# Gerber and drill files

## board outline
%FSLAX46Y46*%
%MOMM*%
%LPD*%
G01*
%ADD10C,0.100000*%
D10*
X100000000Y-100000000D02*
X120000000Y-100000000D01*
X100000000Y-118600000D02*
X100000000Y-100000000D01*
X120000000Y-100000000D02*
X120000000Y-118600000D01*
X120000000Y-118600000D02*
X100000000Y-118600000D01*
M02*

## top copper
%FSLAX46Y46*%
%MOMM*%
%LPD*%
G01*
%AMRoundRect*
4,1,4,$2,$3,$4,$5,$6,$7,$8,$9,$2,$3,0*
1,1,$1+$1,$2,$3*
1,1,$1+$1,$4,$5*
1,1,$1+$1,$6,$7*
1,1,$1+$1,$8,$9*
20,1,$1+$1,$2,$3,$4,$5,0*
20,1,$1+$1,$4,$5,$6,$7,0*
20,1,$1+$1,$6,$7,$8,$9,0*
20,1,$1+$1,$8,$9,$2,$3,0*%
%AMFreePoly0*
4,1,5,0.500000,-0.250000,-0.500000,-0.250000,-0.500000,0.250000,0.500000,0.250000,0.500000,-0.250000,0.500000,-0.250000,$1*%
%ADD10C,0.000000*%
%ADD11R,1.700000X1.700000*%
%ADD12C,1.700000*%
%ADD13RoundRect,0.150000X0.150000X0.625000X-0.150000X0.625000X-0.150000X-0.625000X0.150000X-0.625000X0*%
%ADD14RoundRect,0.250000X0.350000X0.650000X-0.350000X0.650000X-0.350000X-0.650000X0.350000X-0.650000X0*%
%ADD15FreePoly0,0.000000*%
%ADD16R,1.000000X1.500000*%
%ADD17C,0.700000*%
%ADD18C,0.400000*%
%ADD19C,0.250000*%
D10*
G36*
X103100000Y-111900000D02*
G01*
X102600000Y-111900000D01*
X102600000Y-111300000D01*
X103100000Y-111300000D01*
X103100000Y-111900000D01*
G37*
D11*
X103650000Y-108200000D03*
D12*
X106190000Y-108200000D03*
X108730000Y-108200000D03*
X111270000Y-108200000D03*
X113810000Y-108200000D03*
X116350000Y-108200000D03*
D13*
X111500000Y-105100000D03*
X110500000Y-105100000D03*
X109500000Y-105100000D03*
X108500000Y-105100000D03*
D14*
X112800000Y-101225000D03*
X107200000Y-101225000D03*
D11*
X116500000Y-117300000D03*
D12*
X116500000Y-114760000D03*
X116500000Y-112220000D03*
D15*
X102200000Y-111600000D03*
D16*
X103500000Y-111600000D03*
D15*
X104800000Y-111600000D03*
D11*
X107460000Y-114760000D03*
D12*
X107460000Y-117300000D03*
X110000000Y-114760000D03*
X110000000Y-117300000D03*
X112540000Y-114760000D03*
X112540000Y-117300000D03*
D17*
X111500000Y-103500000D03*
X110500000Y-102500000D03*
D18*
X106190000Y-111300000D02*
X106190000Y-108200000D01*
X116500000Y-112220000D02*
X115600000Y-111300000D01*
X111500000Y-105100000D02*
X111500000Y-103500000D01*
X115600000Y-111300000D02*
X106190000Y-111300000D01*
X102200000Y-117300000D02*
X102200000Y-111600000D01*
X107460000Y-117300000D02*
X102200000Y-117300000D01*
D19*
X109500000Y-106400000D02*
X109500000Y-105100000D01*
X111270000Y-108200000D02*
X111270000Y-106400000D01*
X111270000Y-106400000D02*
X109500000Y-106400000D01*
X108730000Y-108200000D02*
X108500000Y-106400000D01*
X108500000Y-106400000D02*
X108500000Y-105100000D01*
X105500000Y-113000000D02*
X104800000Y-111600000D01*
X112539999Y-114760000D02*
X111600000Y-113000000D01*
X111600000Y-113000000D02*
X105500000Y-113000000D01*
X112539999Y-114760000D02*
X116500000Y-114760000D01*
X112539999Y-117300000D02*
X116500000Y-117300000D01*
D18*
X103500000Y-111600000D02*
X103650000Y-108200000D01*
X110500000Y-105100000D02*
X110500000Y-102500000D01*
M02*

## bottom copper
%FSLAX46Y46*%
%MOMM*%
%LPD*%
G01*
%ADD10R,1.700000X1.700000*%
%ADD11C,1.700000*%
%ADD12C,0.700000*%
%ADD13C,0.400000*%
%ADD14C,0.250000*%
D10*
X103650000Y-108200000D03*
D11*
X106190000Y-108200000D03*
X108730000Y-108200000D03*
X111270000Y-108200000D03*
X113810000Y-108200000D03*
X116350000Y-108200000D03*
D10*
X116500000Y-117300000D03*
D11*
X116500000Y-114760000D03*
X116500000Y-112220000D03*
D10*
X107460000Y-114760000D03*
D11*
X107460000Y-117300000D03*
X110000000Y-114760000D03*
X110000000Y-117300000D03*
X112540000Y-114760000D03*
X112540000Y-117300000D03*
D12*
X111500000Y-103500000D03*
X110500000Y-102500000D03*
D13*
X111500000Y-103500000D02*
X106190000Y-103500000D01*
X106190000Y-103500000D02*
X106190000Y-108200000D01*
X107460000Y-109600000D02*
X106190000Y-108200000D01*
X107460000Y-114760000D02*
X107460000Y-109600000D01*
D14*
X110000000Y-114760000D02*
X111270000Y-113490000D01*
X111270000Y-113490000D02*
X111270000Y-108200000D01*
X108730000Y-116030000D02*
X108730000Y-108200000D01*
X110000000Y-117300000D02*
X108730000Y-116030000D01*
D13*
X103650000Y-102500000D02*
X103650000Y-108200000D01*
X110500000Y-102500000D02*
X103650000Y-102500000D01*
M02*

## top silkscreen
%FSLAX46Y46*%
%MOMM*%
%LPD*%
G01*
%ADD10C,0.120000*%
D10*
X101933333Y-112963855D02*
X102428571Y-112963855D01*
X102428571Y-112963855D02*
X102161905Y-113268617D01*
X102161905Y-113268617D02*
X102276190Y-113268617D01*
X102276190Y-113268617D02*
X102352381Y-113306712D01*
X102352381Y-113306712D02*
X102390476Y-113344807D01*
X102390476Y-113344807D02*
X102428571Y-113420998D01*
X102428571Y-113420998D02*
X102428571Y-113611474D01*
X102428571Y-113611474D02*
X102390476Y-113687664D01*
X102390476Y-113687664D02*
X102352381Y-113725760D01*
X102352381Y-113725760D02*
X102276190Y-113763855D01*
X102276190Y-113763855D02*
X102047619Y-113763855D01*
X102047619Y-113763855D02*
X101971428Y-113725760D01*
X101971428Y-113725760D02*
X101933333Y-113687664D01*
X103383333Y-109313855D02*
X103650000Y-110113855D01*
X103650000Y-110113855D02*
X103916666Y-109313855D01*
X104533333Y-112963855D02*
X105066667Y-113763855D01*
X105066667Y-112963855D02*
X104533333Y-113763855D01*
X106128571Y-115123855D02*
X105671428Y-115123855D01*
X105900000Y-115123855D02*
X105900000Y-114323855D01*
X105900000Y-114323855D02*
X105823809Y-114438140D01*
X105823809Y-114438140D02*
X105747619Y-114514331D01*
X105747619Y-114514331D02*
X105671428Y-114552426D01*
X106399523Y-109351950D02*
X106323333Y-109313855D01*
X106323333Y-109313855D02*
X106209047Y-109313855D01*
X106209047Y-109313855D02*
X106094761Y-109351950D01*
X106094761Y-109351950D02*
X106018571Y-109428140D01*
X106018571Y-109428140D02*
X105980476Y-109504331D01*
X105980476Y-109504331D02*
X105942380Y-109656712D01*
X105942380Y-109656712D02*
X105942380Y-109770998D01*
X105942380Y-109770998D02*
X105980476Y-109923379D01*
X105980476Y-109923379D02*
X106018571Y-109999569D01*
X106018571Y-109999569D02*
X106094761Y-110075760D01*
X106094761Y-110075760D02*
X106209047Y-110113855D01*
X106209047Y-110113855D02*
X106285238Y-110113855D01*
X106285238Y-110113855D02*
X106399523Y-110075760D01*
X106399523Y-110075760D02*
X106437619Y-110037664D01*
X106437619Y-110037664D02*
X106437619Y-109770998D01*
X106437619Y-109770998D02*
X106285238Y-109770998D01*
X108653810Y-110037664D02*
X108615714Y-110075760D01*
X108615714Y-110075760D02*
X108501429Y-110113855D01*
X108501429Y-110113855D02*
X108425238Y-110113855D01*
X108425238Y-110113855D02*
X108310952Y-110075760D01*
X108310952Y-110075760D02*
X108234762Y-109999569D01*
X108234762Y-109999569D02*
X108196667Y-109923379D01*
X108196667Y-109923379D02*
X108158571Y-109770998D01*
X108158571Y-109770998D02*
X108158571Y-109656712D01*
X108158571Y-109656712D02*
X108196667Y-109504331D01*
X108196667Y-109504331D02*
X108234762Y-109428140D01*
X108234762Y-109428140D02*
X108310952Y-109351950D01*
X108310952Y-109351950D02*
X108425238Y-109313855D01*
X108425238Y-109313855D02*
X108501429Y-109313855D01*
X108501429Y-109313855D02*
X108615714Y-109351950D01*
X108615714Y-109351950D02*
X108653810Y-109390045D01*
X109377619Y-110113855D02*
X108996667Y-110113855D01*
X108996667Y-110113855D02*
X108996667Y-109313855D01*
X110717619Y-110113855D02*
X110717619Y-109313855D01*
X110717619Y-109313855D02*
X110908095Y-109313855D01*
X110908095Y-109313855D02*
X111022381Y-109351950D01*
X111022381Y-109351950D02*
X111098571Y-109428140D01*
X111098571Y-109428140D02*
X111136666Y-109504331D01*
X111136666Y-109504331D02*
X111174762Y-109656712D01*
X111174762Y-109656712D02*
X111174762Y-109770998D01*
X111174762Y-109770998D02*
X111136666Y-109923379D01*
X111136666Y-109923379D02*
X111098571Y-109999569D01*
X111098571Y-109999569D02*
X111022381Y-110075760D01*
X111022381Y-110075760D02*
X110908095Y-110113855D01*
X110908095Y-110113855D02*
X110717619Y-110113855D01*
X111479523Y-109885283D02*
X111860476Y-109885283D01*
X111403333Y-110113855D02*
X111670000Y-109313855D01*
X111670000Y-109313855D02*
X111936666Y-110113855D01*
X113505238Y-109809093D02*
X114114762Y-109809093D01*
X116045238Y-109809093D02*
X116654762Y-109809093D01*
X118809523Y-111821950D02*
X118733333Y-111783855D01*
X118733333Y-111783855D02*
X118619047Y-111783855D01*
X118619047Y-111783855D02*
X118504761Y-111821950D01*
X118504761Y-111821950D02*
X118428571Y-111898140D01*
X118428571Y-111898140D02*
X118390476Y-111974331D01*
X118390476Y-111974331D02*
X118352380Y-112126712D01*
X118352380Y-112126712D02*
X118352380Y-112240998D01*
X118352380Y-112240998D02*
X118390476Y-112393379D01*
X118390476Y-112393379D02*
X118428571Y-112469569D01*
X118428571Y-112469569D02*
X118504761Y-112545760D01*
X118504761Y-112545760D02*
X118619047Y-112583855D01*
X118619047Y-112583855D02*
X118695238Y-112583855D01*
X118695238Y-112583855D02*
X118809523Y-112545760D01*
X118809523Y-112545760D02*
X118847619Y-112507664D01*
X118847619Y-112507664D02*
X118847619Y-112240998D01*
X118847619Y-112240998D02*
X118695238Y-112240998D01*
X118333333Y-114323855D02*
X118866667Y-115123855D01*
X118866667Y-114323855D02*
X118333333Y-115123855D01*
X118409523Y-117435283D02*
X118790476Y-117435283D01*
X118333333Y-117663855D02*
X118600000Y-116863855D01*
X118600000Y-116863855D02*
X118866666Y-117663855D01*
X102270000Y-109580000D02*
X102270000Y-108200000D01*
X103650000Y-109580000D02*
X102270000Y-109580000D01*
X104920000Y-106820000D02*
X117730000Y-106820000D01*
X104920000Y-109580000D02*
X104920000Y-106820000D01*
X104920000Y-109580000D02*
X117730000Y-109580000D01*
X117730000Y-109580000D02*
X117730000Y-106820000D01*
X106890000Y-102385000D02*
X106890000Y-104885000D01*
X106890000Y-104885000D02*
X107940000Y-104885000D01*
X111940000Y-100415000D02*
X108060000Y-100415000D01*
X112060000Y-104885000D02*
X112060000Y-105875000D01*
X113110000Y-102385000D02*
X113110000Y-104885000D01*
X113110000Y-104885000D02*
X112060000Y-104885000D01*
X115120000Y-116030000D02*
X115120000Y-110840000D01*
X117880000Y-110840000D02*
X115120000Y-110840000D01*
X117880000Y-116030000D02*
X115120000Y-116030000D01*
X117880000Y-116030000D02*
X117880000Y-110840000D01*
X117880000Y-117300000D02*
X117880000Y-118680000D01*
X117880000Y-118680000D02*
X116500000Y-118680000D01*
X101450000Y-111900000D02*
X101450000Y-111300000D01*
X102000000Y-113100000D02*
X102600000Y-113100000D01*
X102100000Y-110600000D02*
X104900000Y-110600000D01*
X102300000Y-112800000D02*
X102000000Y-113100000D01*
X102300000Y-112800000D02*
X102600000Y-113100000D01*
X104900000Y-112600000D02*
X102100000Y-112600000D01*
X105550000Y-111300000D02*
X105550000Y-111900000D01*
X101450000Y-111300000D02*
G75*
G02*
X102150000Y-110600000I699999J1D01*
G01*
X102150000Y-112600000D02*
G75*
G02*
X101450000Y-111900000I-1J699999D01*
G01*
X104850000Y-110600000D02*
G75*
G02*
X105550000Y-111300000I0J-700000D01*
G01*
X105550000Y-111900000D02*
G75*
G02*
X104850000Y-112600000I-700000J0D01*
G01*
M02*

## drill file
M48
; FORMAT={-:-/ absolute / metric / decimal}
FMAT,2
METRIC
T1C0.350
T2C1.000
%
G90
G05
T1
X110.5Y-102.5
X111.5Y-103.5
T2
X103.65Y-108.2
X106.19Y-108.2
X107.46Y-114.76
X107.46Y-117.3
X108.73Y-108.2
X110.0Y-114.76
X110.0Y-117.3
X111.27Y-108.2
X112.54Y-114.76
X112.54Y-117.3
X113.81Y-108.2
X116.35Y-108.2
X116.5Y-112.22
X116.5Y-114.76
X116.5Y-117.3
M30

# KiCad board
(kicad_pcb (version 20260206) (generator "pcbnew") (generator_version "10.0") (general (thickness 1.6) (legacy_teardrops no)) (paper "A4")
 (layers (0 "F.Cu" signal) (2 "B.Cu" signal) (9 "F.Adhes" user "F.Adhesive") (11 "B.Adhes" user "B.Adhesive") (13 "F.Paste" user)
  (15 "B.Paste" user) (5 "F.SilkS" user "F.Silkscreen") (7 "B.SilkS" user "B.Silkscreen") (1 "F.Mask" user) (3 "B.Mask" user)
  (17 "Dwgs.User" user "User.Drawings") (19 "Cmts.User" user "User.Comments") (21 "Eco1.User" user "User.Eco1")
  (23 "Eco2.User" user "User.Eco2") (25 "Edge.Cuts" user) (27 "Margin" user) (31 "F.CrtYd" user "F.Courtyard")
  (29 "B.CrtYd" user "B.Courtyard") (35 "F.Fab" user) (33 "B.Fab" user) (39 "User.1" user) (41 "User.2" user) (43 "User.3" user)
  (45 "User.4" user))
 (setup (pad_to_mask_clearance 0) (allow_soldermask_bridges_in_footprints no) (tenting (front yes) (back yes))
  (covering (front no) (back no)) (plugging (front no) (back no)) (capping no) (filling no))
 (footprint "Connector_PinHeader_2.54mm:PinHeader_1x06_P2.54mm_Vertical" (layer "F.Cu") (at 103.65 108.2 90)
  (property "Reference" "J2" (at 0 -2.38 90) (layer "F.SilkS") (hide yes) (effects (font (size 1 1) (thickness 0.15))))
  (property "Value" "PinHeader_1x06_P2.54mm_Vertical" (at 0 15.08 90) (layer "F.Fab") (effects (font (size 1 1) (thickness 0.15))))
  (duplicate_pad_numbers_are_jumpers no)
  (fp_line (start -1.38 -1.38) (end 0 -1.38) (stroke (width 0.12) (type solid)) (layer "F.SilkS"))
  (fp_line (start -1.38 0) (end -1.38 -1.38) (stroke (width 0.12) (type solid)) (layer "F.SilkS"))
  (fp_line (start 1.38 1.27) (end 1.38 14.08) (stroke (width 0.12) (type solid)) (layer "F.SilkS"))
  (fp_line (start -1.38 1.27) (end 1.38 1.27) (stroke (width 0.12) (type solid)) (layer "F.SilkS"))
  (fp_line (start -1.38 1.27) (end -1.38 14.08) (stroke (width 0.12) (type solid)) (layer "F.SilkS"))
  (fp_line (start -1.38 14.08) (end 1.38 14.08) (stroke (width 0.12) (type solid)) (layer "F.SilkS"))
  (pad "1" thru_hole rect (at 0 0 90) (size 1.7 1.7) (drill 1) (layers "*.Cu" "*.Mask") (remove_unused_layers no) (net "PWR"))
  (pad "2" thru_hole circle (at 0 2.54 90) (size 1.7 1.7) (drill 1) (layers "*.Cu" "*.Mask") (remove_unused_layers no) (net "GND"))
  (pad "3" thru_hole circle (at 0 5.08 90) (size 1.7 1.7) (drill 1) (layers "*.Cu" "*.Mask") (remove_unused_layers no) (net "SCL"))
  (pad "4" thru_hole circle (at 0 7.62 90) (size 1.7 1.7) (drill 1) (layers "*.Cu" "*.Mask") (remove_unused_layers no) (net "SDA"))
  (pad "5" thru_hole circle (at 0 10.16 90) (size 1.7 1.7) (drill 1) (layers "*.Cu" "*.Mask") (remove_unused_layers no))
  (pad "6" thru_hole circle (at 0 12.7 90) (size 1.7 1.7) (drill 1) (layers "*.Cu" "*.Mask") (remove_unused_layers no)))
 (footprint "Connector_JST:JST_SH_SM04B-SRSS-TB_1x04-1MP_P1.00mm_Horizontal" (layer "F.Cu") (at 110 103.1 180)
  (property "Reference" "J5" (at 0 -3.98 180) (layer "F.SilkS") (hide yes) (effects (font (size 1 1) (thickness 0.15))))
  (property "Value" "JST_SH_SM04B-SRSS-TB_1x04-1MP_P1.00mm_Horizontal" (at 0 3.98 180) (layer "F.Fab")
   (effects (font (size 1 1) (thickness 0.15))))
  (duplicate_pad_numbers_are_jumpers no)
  (fp_line (start 3.11 0.715) (end 3.11 -1.785) (stroke (width 0.12) (type solid)) (layer "F.SilkS"))
  (fp_line (start 3.11 -1.785) (end 2.06 -1.785) (stroke (width 0.12) (type solid)) (layer "F.SilkS"))
  (fp_line (start -1.94 2.685) (end 1.94 2.685) (stroke (width 0.12) (type solid)) (layer "F.SilkS"))
  (fp_line (start -2.06 -1.785) (end -2.06 -2.775) (stroke (width 0.12) (type solid)) (layer "F.SilkS"))
  (fp_line (start -3.11 0.715) (end -3.11 -1.785) (stroke (width 0.12) (type solid)) (layer "F.SilkS"))
  (fp_line (start -3.11 -1.785) (end -2.06 -1.785) (stroke (width 0.12) (type solid)) (layer "F.SilkS"))
  (pad "1" smd roundrect (at -1.5 -2 180) (size 0.6 1.55) (layers "F.Cu" "F.Mask" "F.Paste") (roundrect_rratio 0.25) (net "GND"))
  (pad "2" smd roundrect (at -0.5 -2 180) (size 0.6 1.55) (layers "F.Cu" "F.Mask" "F.Paste") (roundrect_rratio 0.25) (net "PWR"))
  (pad "3" smd roundrect (at 0.5 -2 180) (size 0.6 1.55) (layers "F.Cu" "F.Mask" "F.Paste") (roundrect_rratio 0.25) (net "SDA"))
  (pad "4" smd roundrect (at 1.5 -2 180) (size 0.6 1.55) (layers "F.Cu" "F.Mask" "F.Paste") (roundrect_rratio 0.25) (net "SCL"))
  (pad "MP" smd roundrect (at -2.8 1.875 180) (size 1.2 1.8) (layers "F.Cu" "F.Mask" "F.Paste") (roundrect_rratio 0.208333))
  (pad "MP" smd roundrect (at 2.8 1.875 180) (size 1.2 1.8) (layers "F.Cu" "F.Mask" "F.Paste") (roundrect_rratio 0.208333)))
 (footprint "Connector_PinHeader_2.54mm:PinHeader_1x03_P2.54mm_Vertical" (layer "F.Cu") (at 116.5 117.3 180)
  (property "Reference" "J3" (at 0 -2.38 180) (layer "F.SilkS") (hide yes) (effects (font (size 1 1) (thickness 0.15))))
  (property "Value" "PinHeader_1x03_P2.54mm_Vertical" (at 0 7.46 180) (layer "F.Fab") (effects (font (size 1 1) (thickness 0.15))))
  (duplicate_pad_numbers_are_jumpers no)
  (fp_line (start 1.38 1.27) (end 1.38 6.46) (stroke (width 0.12) (type solid)) (layer "F.SilkS"))
  (fp_line (start -1.38 6.46) (end 1.38 6.46) (stroke (width 0.12) (type solid)) (layer "F.SilkS"))
  (fp_line (start -1.38 1.27) (end 1.38 1.27) (stroke (width 0.12) (type solid)) (layer "F.SilkS"))
  (fp_line (start -1.38 1.27) (end -1.38 6.46) (stroke (width 0.12) (type solid)) (layer "F.SilkS"))
  (fp_line (start -1.38 0) (end -1.38 -1.38) (stroke (width 0.12) (type solid)) (layer "F.SilkS"))
  (fp_line (start -1.38 -1.38) (end 0 -1.38) (stroke (width 0.12) (type solid)) (layer "F.SilkS"))
  (pad "1" thru_hole rect (at 0 0 180) (size 1.7 1.7) (drill 1) (layers "*.Cu" "*.Mask") (remove_unused_layers no) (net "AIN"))
  (pad "2" thru_hole circle (at 0 2.54 180) (size 1.7 1.7) (drill 1) (layers "*.Cu" "*.Mask") (remove_unused_layers no) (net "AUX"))
  (pad "3" thru_hole circle (at 0 5.08 180) (size 1.7 1.7) (drill 1) (layers "*.Cu" "*.Mask") (remove_unused_layers no) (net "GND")))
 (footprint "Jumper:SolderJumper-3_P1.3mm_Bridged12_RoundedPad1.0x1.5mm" (layer "F.Cu") (at 103.5 111.6)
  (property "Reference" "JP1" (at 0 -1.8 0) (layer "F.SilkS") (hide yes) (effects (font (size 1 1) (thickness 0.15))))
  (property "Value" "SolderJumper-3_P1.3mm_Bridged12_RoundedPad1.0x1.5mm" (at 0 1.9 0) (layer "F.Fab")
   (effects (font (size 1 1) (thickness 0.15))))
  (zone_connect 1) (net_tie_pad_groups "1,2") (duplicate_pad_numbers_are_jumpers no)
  (fp_poly (pts (xy -0.9 -0.3) (xy -0.4 -0.3) (xy -0.4 0.3) (xy -0.9 0.3)) (stroke (width 0) (type solid)) (fill yes) (layer "F.Cu"))
  (fp_line (start -2.05 0.3) (end -2.05 -0.3) (stroke (width 0.12) (type solid)) (layer "F.SilkS"))
  (fp_line (start -1.5 1.5) (end -0.9 1.5) (stroke (width 0.12) (type solid)) (layer "F.SilkS"))
  (fp_line (start -1.4 -1) (end 1.4 -1) (stroke (width 0.12) (type solid)) (layer "F.SilkS"))
  (fp_line (start -1.2 1.2) (end -1.5 1.5) (stroke (width 0.12) (type solid)) (layer "F.SilkS"))
  (fp_line (start -1.2 1.2) (end -0.9 1.5) (stroke (width 0.12) (type solid)) (layer "F.SilkS"))
  (fp_line (start 1.4 1) (end -1.4 1) (stroke (width 0.12) (type solid)) (layer "F.SilkS"))
  (fp_line (start 2.05 -0.3) (end 2.05 0.3) (stroke (width 0.12) (type solid)) (layer "F.SilkS"))
  (fp_arc (start -2.05 -0.3) (mid -1.844975 -0.794975) (end -1.35 -1) (stroke (width 0.12) (type solid)) (layer "F.SilkS"))
  (fp_arc (start -1.35 1) (mid -1.844975 0.794975) (end -2.05 0.3) (stroke (width 0.12) (type solid)) (layer "F.SilkS"))
  (fp_arc (start 1.35 -1) (mid 1.844975 -0.794975) (end 2.05 -0.3) (stroke (width 0.12) (type solid)) (layer "F.SilkS"))
  (fp_arc (start 2.05 0.3) (mid 1.844975 0.794975) (end 1.35 1) (stroke (width 0.12) (type solid)) (layer "F.SilkS"))
  (pad "1" smd custom (at -1.3 0) (size 1 0.5) (layers "F.Cu" "F.Mask") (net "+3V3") (zone_connect 2) (thermal_bridge_angle 45)
   (options (clearance outline) (anchor rect)) (primitives))
  (pad "2" smd rect (at 0 0) (size 1 1.5) (layers "F.Cu" "F.Mask") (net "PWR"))
  (pad "3" smd custom (at 1.3 0) (size 1 0.5) (layers "F.Cu" "F.Mask") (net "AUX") (zone_connect 2) (thermal_bridge_angle 45)
   (options (clearance outline) (anchor rect)) (primitives)))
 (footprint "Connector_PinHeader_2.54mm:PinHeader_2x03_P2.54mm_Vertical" (layer "B.Cu") (at 107.46 114.76 -90)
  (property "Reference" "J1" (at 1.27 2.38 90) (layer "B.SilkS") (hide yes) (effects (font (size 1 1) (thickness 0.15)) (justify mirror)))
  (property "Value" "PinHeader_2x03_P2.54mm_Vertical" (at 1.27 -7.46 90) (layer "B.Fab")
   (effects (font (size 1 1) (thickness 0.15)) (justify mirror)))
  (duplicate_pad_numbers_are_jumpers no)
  (pad "1" thru_hole rect (at 0 0 270) (size 1.7 1.7) (drill 1) (layers "*.Cu" "*.Mask") (remove_unused_layers no) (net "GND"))
  (pad "2" thru_hole circle (at 2.54 0 270) (size 1.7 1.7) (drill 1) (layers "*.Cu" "*.Mask") (remove_unused_layers no) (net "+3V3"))
  (pad "3" thru_hole circle (at 0 -2.54 270) (size 1.7 1.7) (drill 1) (layers "*.Cu" "*.Mask") (remove_unused_layers no) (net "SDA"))
  (pad "4" thru_hole circle (at 2.54 -2.54 270) (size 1.7 1.7) (drill 1) (layers "*.Cu" "*.Mask") (remove_unused_layers no) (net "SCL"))
  (pad "5" thru_hole circle (at 0 -5.08 270) (size 1.7 1.7) (drill 1) (layers "*.Cu" "*.Mask") (remove_unused_layers no) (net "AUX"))
  (pad "6" thru_hole circle (at 2.54 -5.08 270) (size 1.7 1.7) (drill 1) (layers "*.Cu" "*.Mask") (remove_unused_layers no) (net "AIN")))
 (gr_line (start 100 100) (end 120 100) (stroke (width 0.1) (type default)) (layer "Edge.Cuts"))
 (gr_line (start 100 118.6) (end 100 100) (stroke (width 0.1) (type default)) (layer "Edge.Cuts"))
 (gr_line (start 120 100) (end 120 118.6) (stroke (width 0.1) (type default)) (layer "Edge.Cuts"))
 (gr_line (start 120 118.6) (end 100 118.6) (stroke (width 0.1) (type default)) (layer "Edge.Cuts"))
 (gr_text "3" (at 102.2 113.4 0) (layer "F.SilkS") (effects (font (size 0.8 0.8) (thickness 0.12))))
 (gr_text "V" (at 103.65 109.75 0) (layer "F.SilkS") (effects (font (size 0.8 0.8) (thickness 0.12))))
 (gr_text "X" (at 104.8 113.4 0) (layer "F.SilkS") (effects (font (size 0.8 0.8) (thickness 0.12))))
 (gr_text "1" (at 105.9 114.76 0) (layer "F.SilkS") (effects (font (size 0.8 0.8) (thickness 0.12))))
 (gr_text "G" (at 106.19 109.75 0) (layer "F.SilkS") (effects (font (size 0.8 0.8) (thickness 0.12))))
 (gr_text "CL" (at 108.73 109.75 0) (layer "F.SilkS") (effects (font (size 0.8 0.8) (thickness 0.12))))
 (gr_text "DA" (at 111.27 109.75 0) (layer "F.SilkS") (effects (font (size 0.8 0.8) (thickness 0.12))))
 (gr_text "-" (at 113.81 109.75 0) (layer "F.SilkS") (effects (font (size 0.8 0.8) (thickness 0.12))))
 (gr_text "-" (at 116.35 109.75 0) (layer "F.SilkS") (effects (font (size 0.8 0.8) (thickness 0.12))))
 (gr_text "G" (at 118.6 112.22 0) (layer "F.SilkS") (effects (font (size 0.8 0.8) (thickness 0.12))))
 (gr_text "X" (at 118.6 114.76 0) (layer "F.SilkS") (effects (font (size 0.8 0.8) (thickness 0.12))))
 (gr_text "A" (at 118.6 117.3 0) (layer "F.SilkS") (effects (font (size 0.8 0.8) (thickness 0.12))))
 (segment (start 106.19 111.3) (end 106.19 108.2) (width 0.4) (layer "F.Cu") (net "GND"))
 (segment (start 116.5 112.22) (end 115.6 111.3) (width 0.4) (layer "F.Cu") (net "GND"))
 (segment (start 111.5 105.1) (end 111.5 103.5) (width 0.4) (layer "F.Cu") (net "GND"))
 (segment (start 115.6 111.3) (end 106.19 111.3) (width 0.4) (layer "F.Cu") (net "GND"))
 (via (at 111.5 103.5) (size 0.7) (drill 0.35) (layers "F.Cu" "B.Cu") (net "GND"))
 (segment (start 111.5 103.5) (end 106.19 103.5) (width 0.4) (layer "B.Cu") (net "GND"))
 (segment (start 106.19 103.5) (end 106.19 108.2) (width 0.4) (layer "B.Cu") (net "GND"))
 (segment (start 107.46 109.6) (end 106.19 108.2) (width 0.4) (layer "B.Cu") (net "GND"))
 (segment (start 107.46 114.76) (end 107.46 109.6) (width 0.4) (layer "B.Cu") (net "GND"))
 (segment (start 102.2 117.3) (end 102.2 111.6) (width 0.4) (layer "F.Cu") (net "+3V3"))
 (segment (start 107.46 117.3) (end 102.2 117.3) (width 0.4) (layer "F.Cu") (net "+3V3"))
 (segment (start 109.5 106.4) (end 109.5 105.1) (width 0.25) (layer "F.Cu") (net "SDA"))
 (segment (start 111.27 108.2) (end 111.27 106.4) (width 0.25) (layer "F.Cu") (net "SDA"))
 (segment (start 111.27 106.4) (end 109.5 106.4) (width 0.25) (layer "F.Cu") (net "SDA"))
 (segment (start 110 114.76) (end 111.27 113.49) (width 0.25) (layer "B.Cu") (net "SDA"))
 (segment (start 111.27 113.49) (end 111.27 108.2) (width 0.25) (layer "B.Cu") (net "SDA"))
 (segment (start 108.73 108.2) (end 108.5 106.4) (width 0.25) (layer "F.Cu") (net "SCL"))
 (segment (start 108.5 106.4) (end 108.5 105.1) (width 0.25) (layer "F.Cu") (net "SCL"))
 (segment (start 108.73 116.03) (end 108.73 108.2) (width 0.25) (layer "B.Cu") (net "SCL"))
 (segment (start 110 117.3) (end 108.73 116.03) (width 0.25) (layer "B.Cu") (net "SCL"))
 (segment (start 105.5 113) (end 104.8 111.6) (width 0.25) (layer "F.Cu") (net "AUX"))
 (segment (start 112.539999 114.76) (end 111.6 113) (width 0.25) (layer "F.Cu") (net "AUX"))
 (segment (start 111.6 113) (end 105.5 113) (width 0.25) (layer "F.Cu") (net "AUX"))
 (segment (start 112.539999 114.76) (end 116.5 114.76) (width 0.25) (layer "F.Cu") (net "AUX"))
 (segment (start 112.539999 117.3) (end 116.5 117.3) (width 0.25) (layer "F.Cu") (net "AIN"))
 (segment (start 103.5 111.6) (end 103.65 108.2) (width 0.4) (layer "F.Cu") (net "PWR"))
 (segment (start 110.5 105.1) (end 110.5 102.5) (width 0.4) (layer "F.Cu") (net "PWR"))
 (via (at 110.5 102.5) (size 0.7) (drill 0.35) (layers "F.Cu" "B.Cu") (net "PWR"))
 (segment (start 103.65 102.5) (end 103.65 108.2) (width 0.4) (layer "B.Cu") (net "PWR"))
 (segment (start 110.5 102.5) (end 103.65 102.5) (width 0.4) (layer "B.Cu") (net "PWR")))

